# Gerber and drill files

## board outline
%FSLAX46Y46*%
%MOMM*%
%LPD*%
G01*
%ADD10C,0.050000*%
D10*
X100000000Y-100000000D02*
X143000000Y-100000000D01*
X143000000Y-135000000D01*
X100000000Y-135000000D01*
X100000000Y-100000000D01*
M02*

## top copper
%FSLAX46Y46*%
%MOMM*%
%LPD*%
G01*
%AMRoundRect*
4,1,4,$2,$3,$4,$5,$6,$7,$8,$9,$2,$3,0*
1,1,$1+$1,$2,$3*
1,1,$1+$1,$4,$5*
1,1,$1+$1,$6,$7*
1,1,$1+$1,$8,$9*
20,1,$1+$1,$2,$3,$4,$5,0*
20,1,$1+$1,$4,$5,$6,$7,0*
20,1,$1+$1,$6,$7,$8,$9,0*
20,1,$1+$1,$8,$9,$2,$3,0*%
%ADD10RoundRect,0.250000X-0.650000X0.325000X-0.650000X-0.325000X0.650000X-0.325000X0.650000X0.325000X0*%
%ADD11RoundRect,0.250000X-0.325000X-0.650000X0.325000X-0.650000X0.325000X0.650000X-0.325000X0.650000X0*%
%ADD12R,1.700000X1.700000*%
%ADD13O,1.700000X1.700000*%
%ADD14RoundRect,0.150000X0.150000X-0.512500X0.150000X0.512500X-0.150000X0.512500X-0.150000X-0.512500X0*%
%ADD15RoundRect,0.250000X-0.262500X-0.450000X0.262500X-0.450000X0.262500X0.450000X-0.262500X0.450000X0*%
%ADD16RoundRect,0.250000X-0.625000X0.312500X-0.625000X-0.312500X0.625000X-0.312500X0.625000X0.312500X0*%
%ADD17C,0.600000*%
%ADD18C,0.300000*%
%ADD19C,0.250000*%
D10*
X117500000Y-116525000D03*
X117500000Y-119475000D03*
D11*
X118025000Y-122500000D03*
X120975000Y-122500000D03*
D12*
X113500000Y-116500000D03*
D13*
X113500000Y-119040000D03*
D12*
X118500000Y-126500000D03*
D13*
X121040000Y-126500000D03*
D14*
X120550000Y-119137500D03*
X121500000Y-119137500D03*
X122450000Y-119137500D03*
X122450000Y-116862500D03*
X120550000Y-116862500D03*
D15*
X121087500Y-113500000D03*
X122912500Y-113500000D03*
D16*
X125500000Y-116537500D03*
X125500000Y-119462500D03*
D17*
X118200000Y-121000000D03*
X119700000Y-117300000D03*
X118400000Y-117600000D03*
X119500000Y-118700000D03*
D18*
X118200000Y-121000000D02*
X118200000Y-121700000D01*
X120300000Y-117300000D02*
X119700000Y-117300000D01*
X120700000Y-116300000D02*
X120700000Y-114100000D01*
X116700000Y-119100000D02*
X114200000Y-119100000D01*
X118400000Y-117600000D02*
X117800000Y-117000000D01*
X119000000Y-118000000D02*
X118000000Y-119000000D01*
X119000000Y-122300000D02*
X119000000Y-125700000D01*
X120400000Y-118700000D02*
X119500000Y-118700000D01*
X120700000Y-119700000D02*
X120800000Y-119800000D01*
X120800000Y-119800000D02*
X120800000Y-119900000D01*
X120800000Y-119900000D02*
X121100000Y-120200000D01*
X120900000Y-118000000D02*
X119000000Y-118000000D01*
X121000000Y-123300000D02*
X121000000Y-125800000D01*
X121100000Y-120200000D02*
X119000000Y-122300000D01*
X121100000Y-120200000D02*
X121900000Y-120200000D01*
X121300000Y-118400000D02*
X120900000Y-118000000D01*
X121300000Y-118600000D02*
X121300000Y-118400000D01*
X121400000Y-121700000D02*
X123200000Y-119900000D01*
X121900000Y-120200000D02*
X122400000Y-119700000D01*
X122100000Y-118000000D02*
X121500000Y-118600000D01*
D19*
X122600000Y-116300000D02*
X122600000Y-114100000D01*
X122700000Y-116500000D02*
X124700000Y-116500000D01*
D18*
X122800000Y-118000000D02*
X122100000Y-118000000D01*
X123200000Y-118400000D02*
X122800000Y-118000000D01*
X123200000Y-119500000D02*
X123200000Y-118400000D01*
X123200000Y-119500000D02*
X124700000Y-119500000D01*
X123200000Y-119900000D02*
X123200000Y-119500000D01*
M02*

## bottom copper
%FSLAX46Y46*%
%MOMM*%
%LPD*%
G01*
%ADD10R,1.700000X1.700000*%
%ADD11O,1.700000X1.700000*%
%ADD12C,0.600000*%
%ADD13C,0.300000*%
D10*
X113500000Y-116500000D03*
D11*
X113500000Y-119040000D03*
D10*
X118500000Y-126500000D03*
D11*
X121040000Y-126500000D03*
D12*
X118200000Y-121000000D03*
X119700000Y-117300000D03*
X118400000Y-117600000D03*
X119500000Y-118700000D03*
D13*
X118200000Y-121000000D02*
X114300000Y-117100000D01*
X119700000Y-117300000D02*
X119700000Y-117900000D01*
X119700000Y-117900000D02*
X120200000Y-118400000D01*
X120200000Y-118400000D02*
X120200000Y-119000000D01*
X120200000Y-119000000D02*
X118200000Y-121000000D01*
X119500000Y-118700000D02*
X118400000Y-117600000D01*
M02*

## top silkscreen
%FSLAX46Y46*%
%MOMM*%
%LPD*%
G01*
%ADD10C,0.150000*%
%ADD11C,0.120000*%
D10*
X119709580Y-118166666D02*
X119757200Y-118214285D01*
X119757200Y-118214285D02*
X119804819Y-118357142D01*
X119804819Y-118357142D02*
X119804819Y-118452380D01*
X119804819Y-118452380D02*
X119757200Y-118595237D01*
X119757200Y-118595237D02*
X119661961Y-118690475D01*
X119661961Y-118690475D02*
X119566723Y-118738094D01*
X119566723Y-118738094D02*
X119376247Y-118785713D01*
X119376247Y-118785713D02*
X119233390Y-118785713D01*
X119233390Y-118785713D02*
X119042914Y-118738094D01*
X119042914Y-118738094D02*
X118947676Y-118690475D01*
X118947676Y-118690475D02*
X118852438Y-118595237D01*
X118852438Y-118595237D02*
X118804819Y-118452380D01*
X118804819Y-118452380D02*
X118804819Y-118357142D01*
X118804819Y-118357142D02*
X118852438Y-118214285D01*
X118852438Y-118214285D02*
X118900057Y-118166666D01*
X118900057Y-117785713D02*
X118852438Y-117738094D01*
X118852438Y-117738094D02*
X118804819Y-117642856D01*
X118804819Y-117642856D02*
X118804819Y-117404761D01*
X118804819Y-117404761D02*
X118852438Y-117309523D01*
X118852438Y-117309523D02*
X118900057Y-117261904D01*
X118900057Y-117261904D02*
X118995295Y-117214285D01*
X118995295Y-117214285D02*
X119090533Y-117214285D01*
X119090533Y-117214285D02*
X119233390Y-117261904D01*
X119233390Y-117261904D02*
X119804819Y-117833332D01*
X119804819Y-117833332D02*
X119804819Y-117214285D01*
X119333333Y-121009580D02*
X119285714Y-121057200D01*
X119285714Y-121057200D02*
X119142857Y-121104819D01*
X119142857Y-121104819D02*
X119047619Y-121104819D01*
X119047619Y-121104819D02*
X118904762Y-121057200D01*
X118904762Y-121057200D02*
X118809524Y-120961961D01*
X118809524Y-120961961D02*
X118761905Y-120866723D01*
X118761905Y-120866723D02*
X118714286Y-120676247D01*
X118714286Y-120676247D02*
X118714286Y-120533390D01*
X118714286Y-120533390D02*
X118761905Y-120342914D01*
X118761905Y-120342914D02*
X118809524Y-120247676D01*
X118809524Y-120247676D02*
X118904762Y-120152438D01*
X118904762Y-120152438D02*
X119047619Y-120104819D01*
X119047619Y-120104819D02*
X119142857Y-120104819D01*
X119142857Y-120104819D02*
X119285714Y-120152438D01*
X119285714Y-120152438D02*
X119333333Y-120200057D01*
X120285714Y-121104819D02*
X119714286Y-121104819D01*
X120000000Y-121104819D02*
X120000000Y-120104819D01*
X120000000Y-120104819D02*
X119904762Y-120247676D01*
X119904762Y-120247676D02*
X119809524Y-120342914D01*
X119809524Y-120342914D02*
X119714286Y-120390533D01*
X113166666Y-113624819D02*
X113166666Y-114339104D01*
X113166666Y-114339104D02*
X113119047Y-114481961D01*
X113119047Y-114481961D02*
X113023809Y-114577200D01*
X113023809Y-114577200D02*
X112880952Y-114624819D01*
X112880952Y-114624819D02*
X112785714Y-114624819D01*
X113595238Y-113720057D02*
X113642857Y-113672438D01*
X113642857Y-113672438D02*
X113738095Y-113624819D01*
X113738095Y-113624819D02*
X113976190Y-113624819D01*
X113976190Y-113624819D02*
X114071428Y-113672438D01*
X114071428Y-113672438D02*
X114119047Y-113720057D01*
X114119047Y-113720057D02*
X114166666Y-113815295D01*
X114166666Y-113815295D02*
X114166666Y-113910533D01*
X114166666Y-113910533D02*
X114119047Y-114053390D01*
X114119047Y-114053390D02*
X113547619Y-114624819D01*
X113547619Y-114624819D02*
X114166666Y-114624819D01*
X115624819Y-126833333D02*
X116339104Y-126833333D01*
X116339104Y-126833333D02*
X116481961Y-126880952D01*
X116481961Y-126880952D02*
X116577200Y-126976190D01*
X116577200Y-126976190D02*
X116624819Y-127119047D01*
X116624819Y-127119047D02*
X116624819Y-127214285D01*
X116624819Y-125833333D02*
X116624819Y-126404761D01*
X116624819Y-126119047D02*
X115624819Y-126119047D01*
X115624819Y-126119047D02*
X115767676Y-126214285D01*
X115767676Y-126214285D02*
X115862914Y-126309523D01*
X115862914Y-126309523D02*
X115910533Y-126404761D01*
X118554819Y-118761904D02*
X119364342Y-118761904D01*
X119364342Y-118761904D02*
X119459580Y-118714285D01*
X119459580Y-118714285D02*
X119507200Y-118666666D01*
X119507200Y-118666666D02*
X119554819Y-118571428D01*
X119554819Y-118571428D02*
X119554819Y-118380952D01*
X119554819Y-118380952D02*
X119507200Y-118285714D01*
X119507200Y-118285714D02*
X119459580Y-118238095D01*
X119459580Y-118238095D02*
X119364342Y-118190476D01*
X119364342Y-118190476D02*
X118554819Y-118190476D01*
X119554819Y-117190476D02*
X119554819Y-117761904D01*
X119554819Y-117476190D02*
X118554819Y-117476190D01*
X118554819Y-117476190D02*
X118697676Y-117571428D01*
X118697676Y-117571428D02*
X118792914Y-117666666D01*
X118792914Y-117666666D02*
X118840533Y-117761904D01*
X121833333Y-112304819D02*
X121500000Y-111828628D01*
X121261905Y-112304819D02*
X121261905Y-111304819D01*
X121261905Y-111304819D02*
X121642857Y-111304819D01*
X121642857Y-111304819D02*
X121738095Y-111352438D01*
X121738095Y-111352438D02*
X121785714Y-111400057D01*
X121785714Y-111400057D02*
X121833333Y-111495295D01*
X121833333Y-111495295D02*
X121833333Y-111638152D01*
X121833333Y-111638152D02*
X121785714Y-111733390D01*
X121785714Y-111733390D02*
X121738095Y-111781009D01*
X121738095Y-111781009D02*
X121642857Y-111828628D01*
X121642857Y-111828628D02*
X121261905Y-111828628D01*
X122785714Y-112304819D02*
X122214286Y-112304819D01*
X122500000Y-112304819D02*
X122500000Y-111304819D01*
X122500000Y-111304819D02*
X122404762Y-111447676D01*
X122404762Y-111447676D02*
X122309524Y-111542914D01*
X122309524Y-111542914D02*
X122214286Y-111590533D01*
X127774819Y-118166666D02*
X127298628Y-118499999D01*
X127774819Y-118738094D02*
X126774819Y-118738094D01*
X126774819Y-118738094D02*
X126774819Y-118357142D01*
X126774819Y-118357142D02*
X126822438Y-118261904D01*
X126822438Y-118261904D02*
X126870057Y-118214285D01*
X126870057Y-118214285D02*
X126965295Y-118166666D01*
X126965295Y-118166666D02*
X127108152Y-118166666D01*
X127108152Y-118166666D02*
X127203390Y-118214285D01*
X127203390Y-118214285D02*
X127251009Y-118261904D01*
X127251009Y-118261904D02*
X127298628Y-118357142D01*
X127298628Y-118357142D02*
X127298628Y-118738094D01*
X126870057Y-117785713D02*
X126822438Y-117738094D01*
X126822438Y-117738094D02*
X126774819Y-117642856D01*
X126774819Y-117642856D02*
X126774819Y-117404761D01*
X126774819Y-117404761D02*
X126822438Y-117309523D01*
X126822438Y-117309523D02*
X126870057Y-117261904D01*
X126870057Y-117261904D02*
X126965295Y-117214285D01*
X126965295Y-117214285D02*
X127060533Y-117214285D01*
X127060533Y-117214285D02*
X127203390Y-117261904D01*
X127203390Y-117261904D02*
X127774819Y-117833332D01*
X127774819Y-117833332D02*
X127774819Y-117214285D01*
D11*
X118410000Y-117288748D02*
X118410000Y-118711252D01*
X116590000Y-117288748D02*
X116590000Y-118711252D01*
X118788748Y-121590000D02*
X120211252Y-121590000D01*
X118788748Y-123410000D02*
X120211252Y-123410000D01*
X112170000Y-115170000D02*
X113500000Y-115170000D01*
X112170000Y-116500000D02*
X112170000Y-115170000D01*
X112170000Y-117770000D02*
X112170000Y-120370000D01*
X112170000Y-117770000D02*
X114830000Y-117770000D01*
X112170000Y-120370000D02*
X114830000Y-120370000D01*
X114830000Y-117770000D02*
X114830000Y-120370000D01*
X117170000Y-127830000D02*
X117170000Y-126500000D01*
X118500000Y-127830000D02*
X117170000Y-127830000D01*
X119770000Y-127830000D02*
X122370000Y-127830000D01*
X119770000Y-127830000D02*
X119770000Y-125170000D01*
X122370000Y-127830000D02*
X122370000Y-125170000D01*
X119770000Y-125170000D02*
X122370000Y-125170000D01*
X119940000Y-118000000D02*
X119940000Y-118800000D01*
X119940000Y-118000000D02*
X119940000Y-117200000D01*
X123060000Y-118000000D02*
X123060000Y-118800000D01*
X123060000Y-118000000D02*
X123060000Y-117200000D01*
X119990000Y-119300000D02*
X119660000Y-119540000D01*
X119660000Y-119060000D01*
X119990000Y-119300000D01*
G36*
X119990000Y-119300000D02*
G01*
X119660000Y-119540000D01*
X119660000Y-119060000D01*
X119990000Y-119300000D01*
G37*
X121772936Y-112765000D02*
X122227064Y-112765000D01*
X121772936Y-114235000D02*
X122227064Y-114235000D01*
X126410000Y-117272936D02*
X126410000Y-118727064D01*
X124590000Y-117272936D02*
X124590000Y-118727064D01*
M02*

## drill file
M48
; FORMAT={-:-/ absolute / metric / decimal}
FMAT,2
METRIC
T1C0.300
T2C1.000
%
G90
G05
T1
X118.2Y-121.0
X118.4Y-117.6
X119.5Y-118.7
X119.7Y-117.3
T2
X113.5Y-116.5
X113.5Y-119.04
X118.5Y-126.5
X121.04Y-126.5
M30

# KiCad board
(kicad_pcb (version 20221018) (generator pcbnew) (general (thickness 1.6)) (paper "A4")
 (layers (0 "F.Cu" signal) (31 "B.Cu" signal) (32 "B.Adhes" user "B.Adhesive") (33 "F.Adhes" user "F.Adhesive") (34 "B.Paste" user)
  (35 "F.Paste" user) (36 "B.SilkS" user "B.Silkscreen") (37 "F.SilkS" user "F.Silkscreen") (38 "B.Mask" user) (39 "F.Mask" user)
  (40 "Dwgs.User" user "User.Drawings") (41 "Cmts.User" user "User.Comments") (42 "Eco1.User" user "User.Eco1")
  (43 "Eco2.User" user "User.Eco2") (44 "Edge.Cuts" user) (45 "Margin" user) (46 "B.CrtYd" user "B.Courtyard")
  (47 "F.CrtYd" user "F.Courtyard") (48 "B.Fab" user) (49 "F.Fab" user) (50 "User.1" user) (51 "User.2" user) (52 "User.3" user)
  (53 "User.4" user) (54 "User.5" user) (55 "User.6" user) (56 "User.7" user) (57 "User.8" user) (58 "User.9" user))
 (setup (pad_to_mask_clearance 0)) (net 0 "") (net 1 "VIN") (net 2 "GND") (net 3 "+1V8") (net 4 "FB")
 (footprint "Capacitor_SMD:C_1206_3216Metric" (layer "F.Cu") (at 117.5 118 -90)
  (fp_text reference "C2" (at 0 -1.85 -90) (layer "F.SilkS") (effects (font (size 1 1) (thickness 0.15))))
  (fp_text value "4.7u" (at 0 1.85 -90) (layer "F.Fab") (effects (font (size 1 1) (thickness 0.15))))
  (fp_line (start -0.711252 -0.91) (end 0.711252 -0.91) (stroke (width 0.12) (type solid)) (layer "F.SilkS"))
  (fp_line (start -0.711252 0.91) (end 0.711252 0.91) (stroke (width 0.12) (type solid)) (layer "F.SilkS"))
  (pad "1" smd roundrect (at -1.475 0 270) (size 1.15 1.8) (layers "F.Cu" "F.Paste" "F.Mask") (roundrect_rratio 0.217391) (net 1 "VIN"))
  (pad "2" smd roundrect (at 1.475 0 270) (size 1.15 1.8) (layers "F.Cu" "F.Paste" "F.Mask") (roundrect_rratio 0.217391) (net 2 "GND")))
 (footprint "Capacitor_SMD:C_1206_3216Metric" (layer "F.Cu") (at 119.5 122.5)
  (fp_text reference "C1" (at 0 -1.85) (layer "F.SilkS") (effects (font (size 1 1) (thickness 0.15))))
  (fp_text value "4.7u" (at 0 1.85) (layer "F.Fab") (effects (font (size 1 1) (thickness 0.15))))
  (fp_line (start -0.711252 -0.91) (end 0.711252 -0.91) (stroke (width 0.12) (type solid)) (layer "F.SilkS"))
  (fp_line (start -0.711252 0.91) (end 0.711252 0.91) (stroke (width 0.12) (type solid)) (layer "F.SilkS"))
  (pad "1" smd roundrect (at -1.475 0) (size 1.15 1.8) (layers "F.Cu" "F.Paste" "F.Mask") (roundrect_rratio 0.217391) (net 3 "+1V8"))
  (pad "2" smd roundrect (at 1.475 0) (size 1.15 1.8) (layers "F.Cu" "F.Paste" "F.Mask") (roundrect_rratio 0.217391) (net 2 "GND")))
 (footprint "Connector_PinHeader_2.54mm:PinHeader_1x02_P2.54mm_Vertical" (layer "F.Cu") (at 113.5 116.5)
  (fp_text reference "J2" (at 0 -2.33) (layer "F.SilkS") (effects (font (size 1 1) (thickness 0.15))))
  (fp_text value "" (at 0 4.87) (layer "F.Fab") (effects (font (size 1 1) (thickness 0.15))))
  (fp_line (start -1.33 -1.33) (end 0 -1.33) (stroke (width 0.12) (type solid)) (layer "F.SilkS"))
  (fp_line (start -1.33 0) (end -1.33 -1.33) (stroke (width 0.12) (type solid)) (layer "F.SilkS"))
  (fp_line (start -1.33 1.27) (end -1.33 3.87) (stroke (width 0.12) (type solid)) (layer "F.SilkS"))
  (fp_line (start -1.33 1.27) (end 1.33 1.27) (stroke (width 0.12) (type solid)) (layer "F.SilkS"))
  (fp_line (start -1.33 3.87) (end 1.33 3.87) (stroke (width 0.12) (type solid)) (layer "F.SilkS"))
  (fp_line (start 1.33 1.27) (end 1.33 3.87) (stroke (width 0.12) (type solid)) (layer "F.SilkS"))
  (pad "1" thru_hole rect (at 0 0) (size 1.7 1.7) (drill 1) (layers "*.Cu" "*.Mask") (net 3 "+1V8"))
  (pad "2" thru_hole oval (at 0 2.54) (size 1.7 1.7) (drill 1) (layers "*.Cu" "*.Mask") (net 2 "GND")))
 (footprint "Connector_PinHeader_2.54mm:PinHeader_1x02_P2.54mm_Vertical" (layer "F.Cu") (at 118.5 126.5 90)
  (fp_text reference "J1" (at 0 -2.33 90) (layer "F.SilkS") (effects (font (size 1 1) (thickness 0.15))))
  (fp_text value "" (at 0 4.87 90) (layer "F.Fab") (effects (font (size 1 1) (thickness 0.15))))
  (fp_line (start -1.33 -1.33) (end 0 -1.33) (stroke (width 0.12) (type solid)) (layer "F.SilkS"))
  (fp_line (start -1.33 0) (end -1.33 -1.33) (stroke (width 0.12) (type solid)) (layer "F.SilkS"))
  (fp_line (start -1.33 1.27) (end -1.33 3.87) (stroke (width 0.12) (type solid)) (layer "F.SilkS"))
  (fp_line (start -1.33 1.27) (end 1.33 1.27) (stroke (width 0.12) (type solid)) (layer "F.SilkS"))
  (fp_line (start -1.33 3.87) (end 1.33 3.87) (stroke (width 0.12) (type solid)) (layer "F.SilkS"))
  (fp_line (start 1.33 1.27) (end 1.33 3.87) (stroke (width 0.12) (type solid)) (layer "F.SilkS"))
  (pad "1" thru_hole rect (at 0 0 90) (size 1.7 1.7) (drill 1) (layers "*.Cu" "*.Mask") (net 1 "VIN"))
  (pad "2" thru_hole oval (at 0 2.54 90) (size 1.7 1.7) (drill 1) (layers "*.Cu" "*.Mask") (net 2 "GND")))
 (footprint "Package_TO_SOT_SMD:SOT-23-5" (layer "F.Cu") (at 121.5 118 90)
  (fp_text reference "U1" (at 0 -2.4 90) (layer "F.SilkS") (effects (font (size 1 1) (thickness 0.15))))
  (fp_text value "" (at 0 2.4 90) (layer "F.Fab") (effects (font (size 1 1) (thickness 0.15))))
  (fp_line (start 0 -1.56) (end -0.8 -1.56) (stroke (width 0.12) (type solid)) (layer "F.SilkS"))
  (fp_line (start 0 -1.56) (end 0.8 -1.56) (stroke (width 0.12) (type solid)) (layer "F.SilkS"))
  (fp_line (start 0 1.56) (end -0.8 1.56) (stroke (width 0.12) (type solid)) (layer "F.SilkS"))
  (fp_line (start 0 1.56) (end 0.8 1.56) (stroke (width 0.12) (type solid)) (layer "F.SilkS"))
  (fp_poly
   (pts (xy -1.3 -1.51) (xy -1.54 -1.84) (xy -1.06 -1.84) (xy -1.3 -1.51)) (stroke (width 0.12) (type solid)) (fill solid) (layer "F.SilkS"))
  (pad "1" smd roundrect (at -1.1375 -0.95 90) (size 1.325 0.6) (layers "F.Cu" "F.Paste" "F.Mask") (roundrect_rratio 0.25) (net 1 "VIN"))
  (pad "2" smd roundrect (at -1.1375 0 90) (size 1.325 0.6) (layers "F.Cu" "F.Paste" "F.Mask") (roundrect_rratio 0.25) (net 2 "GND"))
  (pad "3" smd roundrect (at -1.1375 0.95 90) (size 1.325 0.6) (layers "F.Cu" "F.Paste" "F.Mask") (roundrect_rratio 0.25) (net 1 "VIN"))
  (pad "4" smd roundrect (at 1.1375 0.95 90) (size 1.325 0.6) (layers "F.Cu" "F.Paste" "F.Mask") (roundrect_rratio 0.25) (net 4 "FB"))
  (pad "5" smd roundrect (at 1.1375 -0.95 90) (size 1.325 0.6) (layers "F.Cu" "F.Paste" "F.Mask") (roundrect_rratio 0.25) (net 3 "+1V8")))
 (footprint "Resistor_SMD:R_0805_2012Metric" (layer "F.Cu") (at 122 113.5)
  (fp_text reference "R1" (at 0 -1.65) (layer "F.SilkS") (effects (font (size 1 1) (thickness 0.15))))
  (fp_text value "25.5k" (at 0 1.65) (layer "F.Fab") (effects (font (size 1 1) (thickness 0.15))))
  (fp_line (start -0.227064 -0.735) (end 0.227064 -0.735) (stroke (width 0.12) (type solid)) (layer "F.SilkS"))
  (fp_line (start -0.227064 0.735) (end 0.227064 0.735) (stroke (width 0.12) (type solid)) (layer "F.SilkS"))
  (pad "1" smd roundrect (at -0.9125 0) (size 1.025 1.4) (layers "F.Cu" "F.Paste" "F.Mask") (roundrect_rratio 0.243902) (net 3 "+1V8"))
  (pad "2" smd roundrect (at 0.9125 0) (size 1.025 1.4) (layers "F.Cu" "F.Paste" "F.Mask") (roundrect_rratio 0.243902) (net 4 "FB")))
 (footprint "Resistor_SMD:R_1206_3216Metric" (layer "F.Cu") (at 125.5 118 -90)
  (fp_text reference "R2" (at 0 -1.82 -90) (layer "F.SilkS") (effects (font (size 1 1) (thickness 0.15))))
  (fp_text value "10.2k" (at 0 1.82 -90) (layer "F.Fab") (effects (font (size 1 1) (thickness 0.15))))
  (fp_line (start -0.727064 -0.91) (end 0.727064 -0.91) (stroke (width 0.12) (type solid)) (layer "F.SilkS"))
  (fp_line (start -0.727064 0.91) (end 0.727064 0.91) (stroke (width 0.12) (type solid)) (layer "F.SilkS"))
  (pad "1" smd roundrect (at -1.4625 0 270) (size 1.125 1.75) (layers "F.Cu" "F.Paste" "F.Mask") (roundrect_rratio 0.222222) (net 4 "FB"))
  (pad "2" smd roundrect (at 1.4625 0 270) (size 1.125 1.75) (layers "F.Cu" "F.Paste" "F.Mask") (roundrect_rratio 0.222222) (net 2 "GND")))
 (gr_rect (start 100 100) (end 143 135) (stroke (width 0.05) (type default)) (fill none) (layer "Edge.Cuts"))
 (segment (start 118.2 121) (end 118.2 121.7) (width 0.3) (layer "F.Cu") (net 3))
 (segment (start 120.3 117.3) (end 119.7 117.3) (width 0.3) (layer "F.Cu") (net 3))
 (segment (start 120.7 116.3) (end 120.7 114.1) (width 0.3) (layer "F.Cu") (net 3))
 (via (at 118.2 121) (size 0.6) (drill 0.3) (layers "F.Cu" "B.Cu") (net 3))
 (via (at 119.7 117.3) (size 0.6) (drill 0.3) (layers "F.Cu" "B.Cu") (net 3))
 (segment (start 116.7 119.1) (end 114.2 119.1) (width 0.3) (layer "F.Cu") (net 2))
 (segment (start 118.2 121) (end 114.3 117.1) (width 0.3) (layer "B.Cu") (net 3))
 (segment (start 118.4 117.6) (end 117.8 117) (width 0.3) (layer "F.Cu") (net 1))
 (segment (start 119 118) (end 118 119) (width 0.3) (layer "F.Cu") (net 2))
 (segment (start 119 122.3) (end 119 125.7) (width 0.3) (layer "F.Cu") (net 1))
 (segment (start 119.7 117.3) (end 119.7 117.9) (width 0.3) (layer "B.Cu") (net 3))
 (segment (start 119.7 117.9) (end 120.2 118.4) (width 0.3) (layer "B.Cu") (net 3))
 (segment (start 120.2 118.4) (end 120.2 119) (width 0.3) (layer "B.Cu") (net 3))
 (segment (start 120.2 119) (end 118.2 121) (width 0.3) (layer "B.Cu") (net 3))
 (segment (start 120.4 118.7) (end 119.5 118.7) (width 0.3) (layer "F.Cu") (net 1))
 (segment (start 120.7 119.7) (end 120.8 119.8) (width 0.3) (layer "F.Cu") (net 1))
 (segment (start 120.8 119.8) (end 120.8 119.9) (width 0.3) (layer "F.Cu") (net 1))
 (segment (start 120.8 119.9) (end 121.1 120.2) (width 0.3) (layer "F.Cu") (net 1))
 (segment (start 120.9 118) (end 119 118) (width 0.3) (layer "F.Cu") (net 2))
 (segment (start 121 123.3) (end 121 125.8) (width 0.3) (layer "F.Cu") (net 2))
 (segment (start 121.1 120.2) (end 119 122.3) (width 0.3) (layer "F.Cu") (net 1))
 (segment (start 121.1 120.2) (end 121.9 120.2) (width 0.3) (layer "F.Cu") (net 1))
 (segment (start 121.3 118.4) (end 120.9 118) (width 0.3) (layer "F.Cu") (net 2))
 (segment (start 121.3 118.6) (end 121.3 118.4) (width 0.3) (layer "F.Cu") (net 2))
 (segment (start 121.4 121.7) (end 123.2 119.9) (width 0.3) (layer "F.Cu") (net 2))
 (segment (start 121.9 120.2) (end 122.4 119.7) (width 0.3) (layer "F.Cu") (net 1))
 (segment (start 122.1 118) (end 121.5 118.6) (width 0.3) (layer "F.Cu") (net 2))
 (segment (start 122.6 116.3) (end 122.6 114.1) (width 0.25) (layer "F.Cu") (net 4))
 (segment (start 122.7 116.5) (end 124.7 116.5) (width 0.25) (layer "F.Cu") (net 4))
 (segment (start 122.8 118) (end 122.1 118) (width 0.3) (layer "F.Cu") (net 2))
 (segment (start 123.2 118.4) (end 122.8 118) (width 0.3) (layer "F.Cu") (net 2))
 (segment (start 123.2 119.5) (end 123.2 118.4) (width 0.3) (layer "F.Cu") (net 2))
 (segment (start 123.2 119.5) (end 124.7 119.5) (width 0.3) (layer "F.Cu") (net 2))
 (segment (start 123.2 119.9) (end 123.2 119.5) (width 0.3) (layer "F.Cu") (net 2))
 (via (at 118.4 117.6) (size 0.6) (drill 0.3) (layers "F.Cu" "B.Cu") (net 1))
 (via (at 119.5 118.7) (size 0.6) (drill 0.3) (layers "F.Cu" "B.Cu") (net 1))
 (segment (start 119.5 118.7) (end 118.4 117.6) (width 0.3) (layer "B.Cu") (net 1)))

